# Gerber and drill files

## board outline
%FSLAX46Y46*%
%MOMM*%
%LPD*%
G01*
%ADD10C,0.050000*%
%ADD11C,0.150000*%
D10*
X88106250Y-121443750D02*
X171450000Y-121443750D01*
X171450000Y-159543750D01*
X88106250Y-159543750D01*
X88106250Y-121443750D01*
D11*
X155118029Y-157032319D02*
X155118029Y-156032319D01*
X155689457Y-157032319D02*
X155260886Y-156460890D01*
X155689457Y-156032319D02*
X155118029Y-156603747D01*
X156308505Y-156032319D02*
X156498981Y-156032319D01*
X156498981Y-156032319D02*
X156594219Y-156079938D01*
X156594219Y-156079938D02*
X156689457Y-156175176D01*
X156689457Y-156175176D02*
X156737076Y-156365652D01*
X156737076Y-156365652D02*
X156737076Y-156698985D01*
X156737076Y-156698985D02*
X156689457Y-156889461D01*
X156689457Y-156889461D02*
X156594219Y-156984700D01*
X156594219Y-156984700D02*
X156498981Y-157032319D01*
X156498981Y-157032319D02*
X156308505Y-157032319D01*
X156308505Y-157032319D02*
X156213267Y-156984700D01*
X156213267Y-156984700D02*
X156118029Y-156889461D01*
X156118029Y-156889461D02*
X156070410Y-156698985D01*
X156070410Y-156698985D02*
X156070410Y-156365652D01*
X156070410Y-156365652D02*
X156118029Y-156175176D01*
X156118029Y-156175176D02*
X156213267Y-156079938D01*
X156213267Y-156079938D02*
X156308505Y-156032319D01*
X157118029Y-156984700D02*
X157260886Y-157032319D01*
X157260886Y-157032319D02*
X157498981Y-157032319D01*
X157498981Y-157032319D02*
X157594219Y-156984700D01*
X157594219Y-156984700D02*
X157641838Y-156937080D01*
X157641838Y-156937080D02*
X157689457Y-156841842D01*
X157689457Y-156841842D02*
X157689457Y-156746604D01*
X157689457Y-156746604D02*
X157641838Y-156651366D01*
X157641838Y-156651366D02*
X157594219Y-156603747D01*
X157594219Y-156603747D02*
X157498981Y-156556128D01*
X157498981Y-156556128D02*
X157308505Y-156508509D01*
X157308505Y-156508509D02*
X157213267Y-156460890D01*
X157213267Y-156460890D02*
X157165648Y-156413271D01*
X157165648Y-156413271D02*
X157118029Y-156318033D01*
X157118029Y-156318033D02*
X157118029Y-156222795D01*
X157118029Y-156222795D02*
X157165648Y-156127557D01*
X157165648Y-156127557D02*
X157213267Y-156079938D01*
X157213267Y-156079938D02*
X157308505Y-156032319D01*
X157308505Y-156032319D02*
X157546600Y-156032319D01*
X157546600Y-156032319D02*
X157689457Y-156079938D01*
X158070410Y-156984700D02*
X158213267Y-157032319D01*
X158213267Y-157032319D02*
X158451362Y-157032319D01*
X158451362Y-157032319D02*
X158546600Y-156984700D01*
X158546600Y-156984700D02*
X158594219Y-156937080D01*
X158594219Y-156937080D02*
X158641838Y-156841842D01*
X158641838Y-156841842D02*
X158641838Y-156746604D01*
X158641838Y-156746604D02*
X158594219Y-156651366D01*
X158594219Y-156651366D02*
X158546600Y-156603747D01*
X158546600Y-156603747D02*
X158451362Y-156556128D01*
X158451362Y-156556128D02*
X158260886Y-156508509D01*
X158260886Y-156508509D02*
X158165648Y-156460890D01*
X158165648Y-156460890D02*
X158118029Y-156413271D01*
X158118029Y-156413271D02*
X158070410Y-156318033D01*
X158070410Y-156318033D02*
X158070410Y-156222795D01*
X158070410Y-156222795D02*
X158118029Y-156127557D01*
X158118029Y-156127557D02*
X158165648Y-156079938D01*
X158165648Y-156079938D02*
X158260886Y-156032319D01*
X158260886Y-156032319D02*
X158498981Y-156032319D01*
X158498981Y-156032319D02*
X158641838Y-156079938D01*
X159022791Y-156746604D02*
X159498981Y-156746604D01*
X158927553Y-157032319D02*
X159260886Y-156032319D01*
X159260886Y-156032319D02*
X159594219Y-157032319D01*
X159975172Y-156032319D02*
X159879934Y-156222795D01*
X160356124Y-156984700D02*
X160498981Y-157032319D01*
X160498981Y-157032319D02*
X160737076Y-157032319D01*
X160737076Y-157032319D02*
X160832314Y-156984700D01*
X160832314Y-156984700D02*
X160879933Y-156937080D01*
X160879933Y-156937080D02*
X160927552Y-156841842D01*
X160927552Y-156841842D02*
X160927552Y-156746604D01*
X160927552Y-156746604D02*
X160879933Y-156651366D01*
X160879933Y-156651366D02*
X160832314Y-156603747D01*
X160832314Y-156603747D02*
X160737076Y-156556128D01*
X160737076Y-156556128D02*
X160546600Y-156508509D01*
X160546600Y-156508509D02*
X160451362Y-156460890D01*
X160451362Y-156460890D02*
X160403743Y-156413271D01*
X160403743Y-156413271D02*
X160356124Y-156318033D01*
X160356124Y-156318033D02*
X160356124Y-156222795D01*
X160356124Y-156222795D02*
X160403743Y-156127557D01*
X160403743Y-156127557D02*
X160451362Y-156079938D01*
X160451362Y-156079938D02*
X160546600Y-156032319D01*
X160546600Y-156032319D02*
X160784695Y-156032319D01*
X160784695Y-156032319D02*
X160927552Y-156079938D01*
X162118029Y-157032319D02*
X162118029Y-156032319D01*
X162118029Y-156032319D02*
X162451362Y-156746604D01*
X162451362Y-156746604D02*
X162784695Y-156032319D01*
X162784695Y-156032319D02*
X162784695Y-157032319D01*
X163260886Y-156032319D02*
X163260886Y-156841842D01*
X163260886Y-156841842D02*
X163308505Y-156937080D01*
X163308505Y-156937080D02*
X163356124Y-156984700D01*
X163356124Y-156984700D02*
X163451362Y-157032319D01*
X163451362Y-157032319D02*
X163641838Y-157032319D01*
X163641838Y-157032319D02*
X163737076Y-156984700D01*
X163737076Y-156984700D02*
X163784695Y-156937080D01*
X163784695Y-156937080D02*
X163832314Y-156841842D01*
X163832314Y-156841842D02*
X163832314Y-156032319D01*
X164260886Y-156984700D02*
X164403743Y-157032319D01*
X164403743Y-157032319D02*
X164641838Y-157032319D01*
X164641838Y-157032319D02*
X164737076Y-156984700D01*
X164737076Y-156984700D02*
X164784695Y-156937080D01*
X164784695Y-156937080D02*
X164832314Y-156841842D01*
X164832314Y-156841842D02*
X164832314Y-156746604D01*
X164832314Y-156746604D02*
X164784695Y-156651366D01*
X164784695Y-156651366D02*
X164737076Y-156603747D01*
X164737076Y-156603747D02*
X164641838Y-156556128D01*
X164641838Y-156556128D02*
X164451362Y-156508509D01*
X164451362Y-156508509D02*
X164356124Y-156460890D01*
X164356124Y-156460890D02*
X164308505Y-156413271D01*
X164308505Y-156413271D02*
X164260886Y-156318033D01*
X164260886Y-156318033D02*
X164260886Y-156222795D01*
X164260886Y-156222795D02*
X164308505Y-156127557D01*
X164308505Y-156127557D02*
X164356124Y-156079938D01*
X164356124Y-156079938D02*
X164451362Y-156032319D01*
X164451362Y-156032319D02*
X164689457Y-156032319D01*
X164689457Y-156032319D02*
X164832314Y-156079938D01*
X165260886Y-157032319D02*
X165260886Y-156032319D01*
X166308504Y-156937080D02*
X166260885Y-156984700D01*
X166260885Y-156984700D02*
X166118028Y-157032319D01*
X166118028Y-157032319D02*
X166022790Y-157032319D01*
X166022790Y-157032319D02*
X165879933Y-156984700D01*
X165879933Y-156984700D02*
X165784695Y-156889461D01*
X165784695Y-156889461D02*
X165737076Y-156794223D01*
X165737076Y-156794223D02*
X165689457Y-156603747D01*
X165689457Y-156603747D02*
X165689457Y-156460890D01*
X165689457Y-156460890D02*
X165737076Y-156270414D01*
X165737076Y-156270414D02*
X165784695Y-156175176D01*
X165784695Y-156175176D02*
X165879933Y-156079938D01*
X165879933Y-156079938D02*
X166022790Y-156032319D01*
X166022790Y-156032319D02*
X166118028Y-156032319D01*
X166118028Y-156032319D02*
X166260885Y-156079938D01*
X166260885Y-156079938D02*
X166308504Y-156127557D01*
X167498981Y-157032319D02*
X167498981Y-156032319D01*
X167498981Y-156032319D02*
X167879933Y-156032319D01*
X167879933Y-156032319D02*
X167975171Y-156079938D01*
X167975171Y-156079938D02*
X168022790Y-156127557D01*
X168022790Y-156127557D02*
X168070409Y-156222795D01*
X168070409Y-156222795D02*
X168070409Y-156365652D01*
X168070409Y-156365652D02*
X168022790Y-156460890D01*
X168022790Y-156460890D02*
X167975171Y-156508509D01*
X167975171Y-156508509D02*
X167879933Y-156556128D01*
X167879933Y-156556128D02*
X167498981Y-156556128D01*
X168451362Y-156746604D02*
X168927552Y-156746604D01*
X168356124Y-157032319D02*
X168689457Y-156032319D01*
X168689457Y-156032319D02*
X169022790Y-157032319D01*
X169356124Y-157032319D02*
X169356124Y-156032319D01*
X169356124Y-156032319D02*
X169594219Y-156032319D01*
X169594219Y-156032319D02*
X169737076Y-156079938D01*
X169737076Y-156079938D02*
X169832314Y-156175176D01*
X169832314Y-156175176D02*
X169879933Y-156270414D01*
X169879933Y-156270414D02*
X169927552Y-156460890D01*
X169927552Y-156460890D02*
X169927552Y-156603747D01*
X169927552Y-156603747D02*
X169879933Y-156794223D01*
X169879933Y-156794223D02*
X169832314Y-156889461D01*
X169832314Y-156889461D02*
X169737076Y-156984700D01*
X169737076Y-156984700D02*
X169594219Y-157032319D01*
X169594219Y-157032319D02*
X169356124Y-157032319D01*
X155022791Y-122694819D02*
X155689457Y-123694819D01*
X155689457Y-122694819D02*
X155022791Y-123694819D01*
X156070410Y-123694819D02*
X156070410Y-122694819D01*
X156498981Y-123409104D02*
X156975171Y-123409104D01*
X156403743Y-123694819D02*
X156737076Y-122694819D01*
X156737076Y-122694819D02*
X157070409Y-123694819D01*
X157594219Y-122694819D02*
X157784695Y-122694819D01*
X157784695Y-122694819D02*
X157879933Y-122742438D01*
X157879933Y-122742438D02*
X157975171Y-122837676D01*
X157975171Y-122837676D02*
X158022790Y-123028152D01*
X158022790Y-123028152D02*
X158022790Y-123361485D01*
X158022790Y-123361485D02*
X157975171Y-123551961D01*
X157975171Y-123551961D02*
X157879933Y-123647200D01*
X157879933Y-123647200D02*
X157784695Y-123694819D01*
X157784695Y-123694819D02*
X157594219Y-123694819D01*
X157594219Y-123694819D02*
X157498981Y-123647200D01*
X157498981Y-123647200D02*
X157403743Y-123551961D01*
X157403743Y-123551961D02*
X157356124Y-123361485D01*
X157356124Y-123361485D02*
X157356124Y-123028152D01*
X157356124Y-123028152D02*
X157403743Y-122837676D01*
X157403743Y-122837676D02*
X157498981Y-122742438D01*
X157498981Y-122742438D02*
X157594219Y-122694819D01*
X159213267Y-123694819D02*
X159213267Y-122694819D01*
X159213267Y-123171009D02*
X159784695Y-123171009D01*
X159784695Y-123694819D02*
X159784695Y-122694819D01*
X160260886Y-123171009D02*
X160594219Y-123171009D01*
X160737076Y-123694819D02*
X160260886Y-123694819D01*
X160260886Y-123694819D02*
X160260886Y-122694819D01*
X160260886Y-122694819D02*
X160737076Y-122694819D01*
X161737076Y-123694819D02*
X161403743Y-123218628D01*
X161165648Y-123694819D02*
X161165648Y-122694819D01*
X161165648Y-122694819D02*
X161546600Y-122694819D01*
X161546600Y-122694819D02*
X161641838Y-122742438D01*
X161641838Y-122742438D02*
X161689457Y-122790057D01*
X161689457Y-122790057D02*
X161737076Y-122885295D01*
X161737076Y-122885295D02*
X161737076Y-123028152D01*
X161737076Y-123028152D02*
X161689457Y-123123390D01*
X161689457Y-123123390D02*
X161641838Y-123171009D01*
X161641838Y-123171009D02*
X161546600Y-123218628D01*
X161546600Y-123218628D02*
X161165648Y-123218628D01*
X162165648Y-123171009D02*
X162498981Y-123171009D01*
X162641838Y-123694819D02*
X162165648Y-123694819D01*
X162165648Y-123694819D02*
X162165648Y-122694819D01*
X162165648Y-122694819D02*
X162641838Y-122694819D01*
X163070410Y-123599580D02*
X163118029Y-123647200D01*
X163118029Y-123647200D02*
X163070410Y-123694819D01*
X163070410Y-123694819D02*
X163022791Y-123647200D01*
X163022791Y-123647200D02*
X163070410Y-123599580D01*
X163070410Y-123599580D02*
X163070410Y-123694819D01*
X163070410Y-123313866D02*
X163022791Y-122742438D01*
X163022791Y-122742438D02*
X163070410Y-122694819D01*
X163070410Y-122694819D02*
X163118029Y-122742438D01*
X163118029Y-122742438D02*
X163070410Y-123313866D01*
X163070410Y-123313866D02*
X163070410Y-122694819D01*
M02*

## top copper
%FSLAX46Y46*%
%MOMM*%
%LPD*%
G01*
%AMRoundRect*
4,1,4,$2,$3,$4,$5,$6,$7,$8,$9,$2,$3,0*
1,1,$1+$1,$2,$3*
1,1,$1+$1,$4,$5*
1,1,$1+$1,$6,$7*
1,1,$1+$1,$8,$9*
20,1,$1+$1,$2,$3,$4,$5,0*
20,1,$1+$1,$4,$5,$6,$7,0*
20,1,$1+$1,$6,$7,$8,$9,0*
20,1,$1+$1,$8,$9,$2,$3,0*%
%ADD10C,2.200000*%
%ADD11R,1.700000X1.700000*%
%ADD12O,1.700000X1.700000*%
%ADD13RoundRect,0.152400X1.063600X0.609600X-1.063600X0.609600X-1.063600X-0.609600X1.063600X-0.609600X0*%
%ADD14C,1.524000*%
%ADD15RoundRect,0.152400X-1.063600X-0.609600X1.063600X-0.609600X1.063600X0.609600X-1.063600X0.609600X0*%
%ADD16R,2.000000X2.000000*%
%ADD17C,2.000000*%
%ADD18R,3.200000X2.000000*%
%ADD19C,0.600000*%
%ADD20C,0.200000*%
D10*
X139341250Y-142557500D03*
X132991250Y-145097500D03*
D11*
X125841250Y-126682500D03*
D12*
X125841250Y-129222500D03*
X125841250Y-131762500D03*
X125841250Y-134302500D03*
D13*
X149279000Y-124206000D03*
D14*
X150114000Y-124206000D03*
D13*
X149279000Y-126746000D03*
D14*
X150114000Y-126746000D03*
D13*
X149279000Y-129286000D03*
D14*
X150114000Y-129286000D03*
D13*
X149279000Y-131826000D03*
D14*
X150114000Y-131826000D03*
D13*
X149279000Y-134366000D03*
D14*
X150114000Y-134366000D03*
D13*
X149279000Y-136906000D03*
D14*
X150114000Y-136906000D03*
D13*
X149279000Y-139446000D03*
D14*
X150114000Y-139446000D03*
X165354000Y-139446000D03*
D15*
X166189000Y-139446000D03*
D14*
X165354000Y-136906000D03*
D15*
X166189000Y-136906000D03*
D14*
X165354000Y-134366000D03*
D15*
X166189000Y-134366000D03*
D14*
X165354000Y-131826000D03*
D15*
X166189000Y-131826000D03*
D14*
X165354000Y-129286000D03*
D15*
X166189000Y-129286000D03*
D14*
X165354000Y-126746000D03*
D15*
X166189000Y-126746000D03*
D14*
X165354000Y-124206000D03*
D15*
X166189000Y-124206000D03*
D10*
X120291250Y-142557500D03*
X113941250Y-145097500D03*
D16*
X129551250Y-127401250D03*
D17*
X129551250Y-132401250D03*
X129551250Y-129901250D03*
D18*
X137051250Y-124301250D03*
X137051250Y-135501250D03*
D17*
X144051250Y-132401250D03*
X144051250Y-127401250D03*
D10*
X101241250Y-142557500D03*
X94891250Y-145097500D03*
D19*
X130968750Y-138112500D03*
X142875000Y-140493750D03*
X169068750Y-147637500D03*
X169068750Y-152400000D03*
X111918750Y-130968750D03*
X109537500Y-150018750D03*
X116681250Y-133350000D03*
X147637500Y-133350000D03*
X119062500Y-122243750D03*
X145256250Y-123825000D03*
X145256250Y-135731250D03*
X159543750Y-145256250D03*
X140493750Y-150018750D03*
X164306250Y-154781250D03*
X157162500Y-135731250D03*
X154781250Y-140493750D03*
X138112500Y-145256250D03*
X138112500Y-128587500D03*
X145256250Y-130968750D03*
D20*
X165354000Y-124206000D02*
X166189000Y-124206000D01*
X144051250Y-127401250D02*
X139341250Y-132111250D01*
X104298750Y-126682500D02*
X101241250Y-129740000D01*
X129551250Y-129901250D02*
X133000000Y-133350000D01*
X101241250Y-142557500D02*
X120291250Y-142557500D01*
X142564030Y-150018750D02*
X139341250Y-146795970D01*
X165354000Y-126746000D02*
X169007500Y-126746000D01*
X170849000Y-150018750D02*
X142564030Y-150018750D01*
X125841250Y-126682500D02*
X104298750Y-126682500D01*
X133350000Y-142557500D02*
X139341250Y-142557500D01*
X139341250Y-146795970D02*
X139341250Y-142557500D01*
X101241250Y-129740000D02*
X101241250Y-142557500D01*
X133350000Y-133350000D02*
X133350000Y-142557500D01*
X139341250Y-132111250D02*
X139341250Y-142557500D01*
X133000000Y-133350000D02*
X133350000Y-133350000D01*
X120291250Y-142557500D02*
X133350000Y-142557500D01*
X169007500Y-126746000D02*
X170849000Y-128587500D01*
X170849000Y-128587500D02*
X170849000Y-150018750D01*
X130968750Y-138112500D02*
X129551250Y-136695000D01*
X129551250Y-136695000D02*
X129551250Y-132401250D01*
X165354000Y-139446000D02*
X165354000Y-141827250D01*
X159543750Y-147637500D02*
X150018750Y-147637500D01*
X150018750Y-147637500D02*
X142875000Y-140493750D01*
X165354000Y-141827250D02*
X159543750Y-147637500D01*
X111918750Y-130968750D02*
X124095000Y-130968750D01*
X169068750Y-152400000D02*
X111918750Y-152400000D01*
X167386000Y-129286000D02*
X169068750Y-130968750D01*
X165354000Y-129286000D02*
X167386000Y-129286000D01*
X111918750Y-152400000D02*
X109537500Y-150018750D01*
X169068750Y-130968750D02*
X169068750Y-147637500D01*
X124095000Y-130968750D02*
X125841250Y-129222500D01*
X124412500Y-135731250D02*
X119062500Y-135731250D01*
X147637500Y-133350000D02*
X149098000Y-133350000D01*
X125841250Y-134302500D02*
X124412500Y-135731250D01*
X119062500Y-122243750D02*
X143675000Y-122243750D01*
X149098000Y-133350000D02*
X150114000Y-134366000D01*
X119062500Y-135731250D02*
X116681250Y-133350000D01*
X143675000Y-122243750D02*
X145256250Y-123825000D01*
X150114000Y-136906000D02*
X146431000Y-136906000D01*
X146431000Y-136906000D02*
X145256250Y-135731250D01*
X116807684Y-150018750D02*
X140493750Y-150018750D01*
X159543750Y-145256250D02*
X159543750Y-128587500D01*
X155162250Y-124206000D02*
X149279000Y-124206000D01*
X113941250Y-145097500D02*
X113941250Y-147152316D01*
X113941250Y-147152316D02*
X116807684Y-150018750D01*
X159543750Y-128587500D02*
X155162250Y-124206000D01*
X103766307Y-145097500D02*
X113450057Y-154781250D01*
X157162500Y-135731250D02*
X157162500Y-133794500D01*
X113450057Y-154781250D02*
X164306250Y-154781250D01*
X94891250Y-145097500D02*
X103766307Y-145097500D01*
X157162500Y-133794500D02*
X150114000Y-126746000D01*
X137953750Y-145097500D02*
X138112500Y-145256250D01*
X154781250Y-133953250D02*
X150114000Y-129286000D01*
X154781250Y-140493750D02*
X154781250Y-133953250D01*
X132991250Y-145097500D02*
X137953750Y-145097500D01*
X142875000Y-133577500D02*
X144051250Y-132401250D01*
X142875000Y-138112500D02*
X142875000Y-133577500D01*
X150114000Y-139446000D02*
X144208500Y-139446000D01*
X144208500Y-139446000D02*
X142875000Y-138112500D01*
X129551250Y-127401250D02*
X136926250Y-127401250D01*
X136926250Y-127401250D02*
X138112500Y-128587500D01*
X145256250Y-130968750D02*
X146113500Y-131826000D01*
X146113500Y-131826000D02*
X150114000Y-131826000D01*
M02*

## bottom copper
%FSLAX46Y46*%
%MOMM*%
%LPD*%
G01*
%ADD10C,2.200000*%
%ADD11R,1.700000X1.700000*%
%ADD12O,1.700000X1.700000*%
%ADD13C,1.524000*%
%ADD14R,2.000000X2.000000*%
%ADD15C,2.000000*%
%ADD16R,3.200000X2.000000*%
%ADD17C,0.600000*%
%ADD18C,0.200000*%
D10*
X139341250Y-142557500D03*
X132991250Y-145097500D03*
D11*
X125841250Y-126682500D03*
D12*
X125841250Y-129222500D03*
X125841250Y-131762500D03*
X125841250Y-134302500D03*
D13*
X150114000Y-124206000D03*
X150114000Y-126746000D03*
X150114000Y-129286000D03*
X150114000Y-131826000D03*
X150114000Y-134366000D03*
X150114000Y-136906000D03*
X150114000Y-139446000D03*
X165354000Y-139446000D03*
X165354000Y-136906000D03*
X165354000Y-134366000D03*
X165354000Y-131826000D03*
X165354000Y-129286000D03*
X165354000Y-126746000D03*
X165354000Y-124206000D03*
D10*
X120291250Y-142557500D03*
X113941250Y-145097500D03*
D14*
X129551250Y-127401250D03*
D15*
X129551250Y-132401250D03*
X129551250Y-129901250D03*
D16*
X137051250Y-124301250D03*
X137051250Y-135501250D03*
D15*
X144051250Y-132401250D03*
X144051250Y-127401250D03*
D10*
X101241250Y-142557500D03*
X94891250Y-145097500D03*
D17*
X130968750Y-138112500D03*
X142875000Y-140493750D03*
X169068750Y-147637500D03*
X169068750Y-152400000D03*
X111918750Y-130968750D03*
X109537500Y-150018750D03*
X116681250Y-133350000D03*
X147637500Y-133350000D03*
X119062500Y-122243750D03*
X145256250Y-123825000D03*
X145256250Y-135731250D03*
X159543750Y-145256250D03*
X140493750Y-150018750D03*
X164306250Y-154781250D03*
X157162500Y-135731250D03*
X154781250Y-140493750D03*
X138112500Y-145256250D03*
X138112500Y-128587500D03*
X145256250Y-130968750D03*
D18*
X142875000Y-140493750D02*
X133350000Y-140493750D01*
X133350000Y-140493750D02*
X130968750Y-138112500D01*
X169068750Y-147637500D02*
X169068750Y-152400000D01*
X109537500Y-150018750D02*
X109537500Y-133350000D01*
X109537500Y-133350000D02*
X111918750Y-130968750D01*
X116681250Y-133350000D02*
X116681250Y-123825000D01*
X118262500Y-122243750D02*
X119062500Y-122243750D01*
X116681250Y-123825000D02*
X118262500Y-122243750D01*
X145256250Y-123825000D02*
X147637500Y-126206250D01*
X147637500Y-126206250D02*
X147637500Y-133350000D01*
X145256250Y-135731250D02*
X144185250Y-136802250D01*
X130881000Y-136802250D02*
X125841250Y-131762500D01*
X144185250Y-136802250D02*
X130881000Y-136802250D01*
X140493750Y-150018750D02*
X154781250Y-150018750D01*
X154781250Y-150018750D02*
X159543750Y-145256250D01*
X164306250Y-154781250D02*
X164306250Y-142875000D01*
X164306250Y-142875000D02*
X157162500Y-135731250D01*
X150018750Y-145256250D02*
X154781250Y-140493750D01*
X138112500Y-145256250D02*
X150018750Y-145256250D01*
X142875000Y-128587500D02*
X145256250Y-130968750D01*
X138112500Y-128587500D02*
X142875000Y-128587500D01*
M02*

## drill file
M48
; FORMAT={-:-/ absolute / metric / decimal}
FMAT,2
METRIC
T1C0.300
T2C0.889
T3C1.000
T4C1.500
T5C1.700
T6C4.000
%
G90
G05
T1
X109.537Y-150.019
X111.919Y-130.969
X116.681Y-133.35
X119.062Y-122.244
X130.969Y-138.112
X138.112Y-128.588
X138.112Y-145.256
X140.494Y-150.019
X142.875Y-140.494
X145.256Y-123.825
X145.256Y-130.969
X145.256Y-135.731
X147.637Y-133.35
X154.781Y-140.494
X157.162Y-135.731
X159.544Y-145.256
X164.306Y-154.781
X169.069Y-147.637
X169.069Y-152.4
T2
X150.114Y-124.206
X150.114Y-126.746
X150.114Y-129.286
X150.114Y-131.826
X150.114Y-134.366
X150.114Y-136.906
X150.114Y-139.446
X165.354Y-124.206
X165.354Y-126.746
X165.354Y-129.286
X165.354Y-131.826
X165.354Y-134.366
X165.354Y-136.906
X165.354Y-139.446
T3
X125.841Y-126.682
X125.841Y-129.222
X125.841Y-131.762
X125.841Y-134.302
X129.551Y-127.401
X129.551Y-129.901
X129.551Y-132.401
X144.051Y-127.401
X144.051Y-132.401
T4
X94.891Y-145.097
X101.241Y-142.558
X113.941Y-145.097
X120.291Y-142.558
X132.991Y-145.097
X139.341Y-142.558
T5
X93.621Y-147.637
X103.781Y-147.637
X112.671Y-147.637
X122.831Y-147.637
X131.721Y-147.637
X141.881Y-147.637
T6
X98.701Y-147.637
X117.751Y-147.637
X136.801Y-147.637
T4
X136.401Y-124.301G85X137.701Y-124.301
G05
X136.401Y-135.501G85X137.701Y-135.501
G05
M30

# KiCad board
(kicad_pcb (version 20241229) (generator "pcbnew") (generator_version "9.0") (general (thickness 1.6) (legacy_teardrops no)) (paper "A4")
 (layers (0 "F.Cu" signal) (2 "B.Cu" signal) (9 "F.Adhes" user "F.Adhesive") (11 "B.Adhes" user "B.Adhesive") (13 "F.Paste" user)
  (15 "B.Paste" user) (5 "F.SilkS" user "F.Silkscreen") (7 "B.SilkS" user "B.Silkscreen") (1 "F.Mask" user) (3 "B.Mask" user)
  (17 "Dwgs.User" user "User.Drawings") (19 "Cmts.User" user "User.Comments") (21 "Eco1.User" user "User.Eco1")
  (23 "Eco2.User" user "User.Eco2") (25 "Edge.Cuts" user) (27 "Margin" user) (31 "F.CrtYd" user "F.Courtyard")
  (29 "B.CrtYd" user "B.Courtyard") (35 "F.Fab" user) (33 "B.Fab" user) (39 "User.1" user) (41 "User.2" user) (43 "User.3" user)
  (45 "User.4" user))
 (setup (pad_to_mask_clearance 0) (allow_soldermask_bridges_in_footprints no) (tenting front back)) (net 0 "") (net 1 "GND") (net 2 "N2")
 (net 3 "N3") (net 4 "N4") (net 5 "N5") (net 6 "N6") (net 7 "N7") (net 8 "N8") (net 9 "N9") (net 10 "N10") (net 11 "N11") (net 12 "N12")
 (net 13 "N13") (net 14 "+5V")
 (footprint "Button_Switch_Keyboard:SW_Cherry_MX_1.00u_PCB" (layer "F.Cu") (at 139.34125 142.5575)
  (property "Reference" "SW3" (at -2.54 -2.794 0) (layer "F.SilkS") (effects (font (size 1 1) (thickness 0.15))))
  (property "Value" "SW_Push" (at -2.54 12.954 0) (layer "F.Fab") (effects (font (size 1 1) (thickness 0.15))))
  (pad "" np_thru_hole circle (at -7.62 5.08) (size 1.7 1.7) (drill 1.7) (layers "*.Cu" "*.Mask"))
  (pad "" np_thru_hole circle (at -2.54 5.08) (size 4 4) (drill 4) (layers "*.Cu" "*.Mask"))
  (pad "" np_thru_hole circle (at 2.54 5.08) (size 1.7 1.7) (drill 1.7) (layers "*.Cu" "*.Mask"))
  (pad "1" thru_hole circle (at 0 0) (size 2.2 2.2) (drill 1.5) (layers "*.Cu" "*.Mask") (remove_unused_layers no) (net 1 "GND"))
  (pad "2" thru_hole circle (at -6.35 2.54) (size 2.2 2.2) (drill 1.5) (layers "*.Cu" "*.Mask") (remove_unused_layers no) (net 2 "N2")))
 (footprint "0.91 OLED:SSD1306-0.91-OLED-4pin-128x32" (layer "F.Cu") (at 89.34125 124.4925)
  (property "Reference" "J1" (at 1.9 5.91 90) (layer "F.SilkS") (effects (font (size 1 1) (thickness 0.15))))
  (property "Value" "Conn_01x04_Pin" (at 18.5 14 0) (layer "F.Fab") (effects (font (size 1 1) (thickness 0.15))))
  (pad "1" thru_hole rect (at 36.5 2.19) (size 1.7 1.7) (drill 1) (layers "*.Cu" "*.Mask") (remove_unused_layers no) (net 1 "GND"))
  (pad "2" thru_hole oval (at 36.5 4.73) (size 1.7 1.7) (drill 1) (layers "*.Cu" "*.Mask") (remove_unused_layers no) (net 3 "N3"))
  (pad "3" thru_hole oval (at 36.5 7.27) (size 1.7 1.7) (drill 1) (layers "*.Cu" "*.Mask") (remove_unused_layers no) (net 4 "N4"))
  (pad "4" thru_hole oval (at 36.5 9.81) (size 1.7 1.7) (drill 1) (layers "*.Cu" "*.Mask") (remove_unused_layers no) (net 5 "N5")))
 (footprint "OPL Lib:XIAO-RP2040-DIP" (layer "F.Cu") (at 157.734 131.826)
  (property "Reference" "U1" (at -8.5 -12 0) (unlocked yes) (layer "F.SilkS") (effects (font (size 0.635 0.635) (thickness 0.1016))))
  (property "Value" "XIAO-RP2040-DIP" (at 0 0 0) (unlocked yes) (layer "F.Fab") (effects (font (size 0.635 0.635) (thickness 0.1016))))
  (pad "1" smd roundrect (at -8.455 -7.62 180) (size 2.432 1.524) (layers "F.Cu" "F.Mask") (roundrect_rratio 0.1) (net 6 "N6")
   (thermal_bridge_angle 45))
  (pad "1" thru_hole circle (at -7.62 -7.62 180) (size 1.524 1.524) (drill 0.889) (layers "*.Cu" "*.Mask") (remove_unused_layers no)
   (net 6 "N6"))
  (pad "2" smd roundrect (at -8.455 -5.08 180) (size 2.432 1.524) (layers "F.Cu" "F.Mask") (roundrect_rratio 0.1) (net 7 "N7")
   (thermal_bridge_angle 45))
  (pad "2" thru_hole circle (at -7.62 -5.08 180) (size 1.524 1.524) (drill 0.889) (layers "*.Cu" "*.Mask") (remove_unused_layers no)
   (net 7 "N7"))
  (pad "3" smd roundrect (at -8.455 -2.54 180) (size 2.432 1.524) (layers "F.Cu" "F.Mask") (roundrect_rratio 0.1) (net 2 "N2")
   (thermal_bridge_angle 45))
  (pad "3" thru_hole circle (at -7.62 -2.54 180) (size 1.524 1.524) (drill 0.889) (layers "*.Cu" "*.Mask") (remove_unused_layers no)
   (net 2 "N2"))
  (pad "4" smd roundrect (at -8.455 0 180) (size 2.432 1.524) (layers "F.Cu" "F.Mask") (roundrect_rratio 0.1) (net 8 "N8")
   (thermal_bridge_angle 45))
  (pad "4" thru_hole circle (at -7.62 0 180) (size 1.524 1.524) (drill 0.889) (layers "*.Cu" "*.Mask") (remove_unused_layers no)
   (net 8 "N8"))
  (pad "5" smd roundrect (at -8.455 2.54 180) (size 2.432 1.524) (layers "F.Cu" "F.Mask") (roundrect_rratio 0.1) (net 5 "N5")
   (thermal_bridge_angle 45))
  (pad "5" thru_hole circle (at -7.62 2.54 180) (size 1.524 1.524) (drill 0.889) (layers "*.Cu" "*.Mask") (remove_unused_layers no)
   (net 5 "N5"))
  (pad "6" smd roundrect (at -8.455 5.08 180) (size 2.432 1.524) (layers "F.Cu" "F.Mask") (roundrect_rratio 0.1) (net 4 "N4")
   (thermal_bridge_angle 45))
  (pad "6" thru_hole circle (at -7.62 5.08 180) (size 1.524 1.524) (drill 0.889) (layers "*.Cu" "*.Mask") (remove_unused_layers no)
   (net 4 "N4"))
  (pad "7" smd roundrect (at -8.455 7.62 180) (size 2.432 1.524) (layers "F.Cu" "F.Mask") (roundrect_rratio 0.1) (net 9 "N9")
   (thermal_bridge_angle 45))
  (pad "7" thru_hole circle (at -7.62 7.62 180) (size 1.524 1.524) (drill 0.889) (layers "*.Cu" "*.Mask") (remove_unused_layers no)
   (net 9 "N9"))
  (pad "8" thru_hole circle (at 7.62 7.62) (size 1.524 1.524) (drill 0.889) (layers "*.Cu" "*.Mask") (remove_unused_layers no)
   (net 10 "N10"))
  (pad "8" smd roundrect (at 8.455 7.62) (size 2.432 1.524) (layers "F.Cu" "F.Mask") (roundrect_rratio 0.1) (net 10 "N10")
   (thermal_bridge_angle 45))
  (pad "9" thru_hole circle (at 7.62 5.08) (size 1.524 1.524) (drill 0.889) (layers "*.Cu" "*.Mask") (remove_unused_layers no)
   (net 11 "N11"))
  (pad "9" smd roundrect (at 8.455 5.08) (size 2.432 1.524) (layers "F.Cu" "F.Mask") (roundrect_rratio 0.1) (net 11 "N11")
   (thermal_bridge_angle 45))
  (pad "10" thru_hole circle (at 7.62 2.54) (size 1.524 1.524) (drill 0.889) (layers "*.Cu" "*.Mask") (remove_unused_layers no)
   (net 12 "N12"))
  (pad "10" smd roundrect (at 8.455 2.54) (size 2.432 1.524) (layers "F.Cu" "F.Mask") (roundrect_rratio 0.1) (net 12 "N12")
   (thermal_bridge_angle 45))
  (pad "11" thru_hole circle (at 7.62 0) (size 1.524 1.524) (drill 0.889) (layers "*.Cu" "*.Mask") (remove_unused_layers no) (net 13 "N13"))
  (pad "11" smd roundrect (at 8.455 0) (size 2.432 1.524) (layers "F.Cu" "F.Mask") (roundrect_rratio 0.1) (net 13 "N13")
   (thermal_bridge_angle 45))
  (pad "12" thru_hole circle (at 7.62 -2.54) (size 1.524 1.524) (drill 0.889) (layers "*.Cu" "*.Mask") (remove_unused_layers no)
   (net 3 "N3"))
  (pad "12" smd roundrect (at 8.455 -2.54) (size 2.432 1.524) (layers "F.Cu" "F.Mask") (roundrect_rratio 0.1) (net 3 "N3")
   (thermal_bridge_angle 45))
  (pad "13" thru_hole circle (at 7.62 -5.08) (size 1.524 1.524) (drill 0.889) (layers "*.Cu" "*.Mask") (remove_unused_layers no)
   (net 1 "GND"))
  (pad "13" smd roundrect (at 8.455 -5.08) (size 2.432 1.524) (layers "F.Cu" "F.Mask") (roundrect_rratio 0.1) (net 1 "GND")
   (thermal_bridge_angle 45))
  (pad "14" thru_hole circle (at 7.62 -7.62) (size 1.524 1.524) (drill 0.889) (layers "*.Cu" "*.Mask") (remove_unused_layers no)
   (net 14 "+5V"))
  (pad "14" smd roundrect (at 8.455 -7.62) (size 2.432 1.524) (layers "F.Cu" "F.Mask") (roundrect_rratio 0.1) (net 14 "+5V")
   (thermal_bridge_angle 45)))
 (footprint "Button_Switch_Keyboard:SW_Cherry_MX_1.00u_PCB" (layer "F.Cu") (at 120.29125 142.5575)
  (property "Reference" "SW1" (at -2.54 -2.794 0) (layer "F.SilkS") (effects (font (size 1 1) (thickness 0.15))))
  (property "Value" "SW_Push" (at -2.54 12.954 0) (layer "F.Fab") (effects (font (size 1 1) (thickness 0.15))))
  (pad "" np_thru_hole circle (at -7.62 5.08) (size 1.7 1.7) (drill 1.7) (layers "*.Cu" "*.Mask"))
  (pad "" np_thru_hole circle (at -2.54 5.08) (size 4 4) (drill 4) (layers "*.Cu" "*.Mask"))
  (pad "" np_thru_hole circle (at 2.54 5.08) (size 1.7 1.7) (drill 1.7) (layers "*.Cu" "*.Mask"))
  (pad "1" thru_hole circle (at 0 0) (size 2.2 2.2) (drill 1.5) (layers "*.Cu" "*.Mask") (remove_unused_layers no) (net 1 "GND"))
  (pad "2" thru_hole circle (at -6.35 2.54) (size 2.2 2.2) (drill 1.5) (layers "*.Cu" "*.Mask") (remove_unused_layers no) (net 6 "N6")))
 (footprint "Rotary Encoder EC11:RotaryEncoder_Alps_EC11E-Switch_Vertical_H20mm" (layer "F.Cu") (at 129.55125 127.40125)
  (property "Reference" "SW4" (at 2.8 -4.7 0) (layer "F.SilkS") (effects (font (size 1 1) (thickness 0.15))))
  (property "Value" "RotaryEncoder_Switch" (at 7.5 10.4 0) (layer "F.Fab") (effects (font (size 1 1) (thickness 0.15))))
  (pad "A" thru_hole rect (at 0 0) (size 2 2) (drill 1) (layers "*.Cu" "*.Mask") (remove_unused_layers no) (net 8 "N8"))
  (pad "B" thru_hole circle (at 0 5) (size 2 2) (drill 1) (layers "*.Cu" "*.Mask") (remove_unused_layers no) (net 10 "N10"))
  (pad "C" thru_hole circle (at 0 2.5) (size 2 2) (drill 1) (layers "*.Cu" "*.Mask") (remove_unused_layers no) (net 1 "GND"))
  (pad "MP" thru_hole rect (at 7.5 -3.1) (size 3.2 2) (drill oval 2.8 1.5) (layers "*.Cu" "*.Mask") (remove_unused_layers no))
  (pad "MP" thru_hole rect (at 7.5 8.1) (size 3.2 2) (drill oval 2.8 1.5) (layers "*.Cu" "*.Mask") (remove_unused_layers no))
  (pad "S1" thru_hole circle (at 14.5 5) (size 2 2) (drill 1) (layers "*.Cu" "*.Mask") (remove_unused_layers no) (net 9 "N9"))
  (pad "S2" thru_hole circle (at 14.5 0) (size 2 2) (drill 1) (layers "*.Cu" "*.Mask") (remove_unused_layers no) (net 1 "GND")))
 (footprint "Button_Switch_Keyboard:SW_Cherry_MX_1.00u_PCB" (layer "F.Cu") (at 101.24125 142.5575)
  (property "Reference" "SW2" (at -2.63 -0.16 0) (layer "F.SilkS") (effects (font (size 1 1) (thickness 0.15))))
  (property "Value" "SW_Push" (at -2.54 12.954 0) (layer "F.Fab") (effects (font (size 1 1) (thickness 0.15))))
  (pad "" np_thru_hole circle (at -7.62 5.08) (size 1.7 1.7) (drill 1.7) (layers "*.Cu" "*.Mask"))
  (pad "" np_thru_hole circle (at -2.54 5.08) (size 4 4) (drill 4) (layers "*.Cu" "*.Mask"))
  (pad "" np_thru_hole circle (at 2.54 5.08) (size 1.7 1.7) (drill 1.7) (layers "*.Cu" "*.Mask"))
  (pad "1" thru_hole circle (at 0 0) (size 2.2 2.2) (drill 1.5) (layers "*.Cu" "*.Mask") (remove_unused_layers no) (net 1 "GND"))
  (pad "2" thru_hole circle (at -6.35 2.54) (size 2.2 2.2) (drill 1.5) (layers "*.Cu" "*.Mask") (remove_unused_layers no) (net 7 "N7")))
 (gr_rect (start 88.10625 121.44375) (end 171.45 159.54375) (stroke (width 0.05) (type default)) (fill no) (layer "Edge.Cuts"))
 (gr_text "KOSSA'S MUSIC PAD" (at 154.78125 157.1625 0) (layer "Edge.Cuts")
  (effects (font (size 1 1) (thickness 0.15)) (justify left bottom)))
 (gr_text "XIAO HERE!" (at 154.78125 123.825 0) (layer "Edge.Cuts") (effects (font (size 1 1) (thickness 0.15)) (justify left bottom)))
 (segment (start 165.354 124.206) (end 166.189 124.206) (width 0.2) (layer "F.Cu") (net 14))
 (segment (start 144.05125 127.40125) (end 139.34125 132.11125) (width 0.2) (layer "F.Cu") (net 1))
 (segment (start 104.29875 126.6825) (end 101.24125 129.74) (width 0.2) (layer "F.Cu") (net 1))
 (segment (start 129.55125 129.90125) (end 133 133.35) (width 0.2) (layer "F.Cu") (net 1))
 (segment (start 101.24125 142.5575) (end 120.29125 142.5575) (width 0.2) (layer "F.Cu") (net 1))
 (segment (start 142.56403 150.01875) (end 139.34125 146.79597) (width 0.2) (layer "F.Cu") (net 1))
 (segment (start 165.354 126.746) (end 169.0075 126.746) (width 0.2) (layer "F.Cu") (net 1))
 (segment (start 170.849 150.01875) (end 142.56403 150.01875) (width 0.2) (layer "F.Cu") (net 1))
 (segment (start 125.84125 126.6825) (end 104.29875 126.6825) (width 0.2) (layer "F.Cu") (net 1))
 (segment (start 133.35 142.5575) (end 139.34125 142.5575) (width 0.2) (layer "F.Cu") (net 1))
 (segment (start 139.34125 146.79597) (end 139.34125 142.5575) (width 0.2) (layer "F.Cu") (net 1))
 (segment (start 101.24125 129.74) (end 101.24125 142.5575) (width 0.2) (layer "F.Cu") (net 1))
 (segment (start 133.35 133.35) (end 133.35 142.5575) (width 0.2) (layer "F.Cu") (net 1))
 (segment (start 139.34125 132.11125) (end 139.34125 142.5575) (width 0.2) (layer "F.Cu") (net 1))
 (segment (start 133 133.35) (end 133.35 133.35) (width 0.2) (layer "F.Cu") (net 1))
 (segment (start 120.29125 142.5575) (end 133.35 142.5575) (width 0.2) (layer "F.Cu") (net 1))
 (segment (start 169.0075 126.746) (end 170.849 128.5875) (width 0.2) (layer "F.Cu") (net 1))
 (segment (start 170.849 128.5875) (end 170.849 150.01875) (width 0.2) (layer "F.Cu") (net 1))
 (segment (start 130.96875 138.1125) (end 129.55125 136.695) (width 0.2) (layer "F.Cu") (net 10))
 (segment (start 129.55125 136.695) (end 129.55125 132.40125) (width 0.2) (layer "F.Cu") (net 10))
 (segment (start 165.354 139.446) (end 165.354 141.82725) (width 0.2) (layer "F.Cu") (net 10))
 (segment (start 159.54375 147.6375) (end 150.01875 147.6375) (width 0.2) (layer "F.Cu") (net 10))
 (segment (start 150.01875 147.6375) (end 142.875 140.49375) (width 0.2) (layer "F.Cu") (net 10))
 (segment (start 165.354 141.82725) (end 159.54375 147.6375) (width 0.2) (layer "F.Cu") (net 10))
 (via (at 130.96875 138.1125) (size 0.6) (drill 0.3) (layers "F.Cu" "B.Cu") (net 10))
 (via (at 142.875 140.49375) (size 0.6) (drill 0.3) (layers "F.Cu" "B.Cu") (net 10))
 (segment (start 142.875 140.49375) (end 133.35 140.49375) (width 0.2) (layer "B.Cu") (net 10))
 (segment (start 133.35 140.49375) (end 130.96875 138.1125) (width 0.2) (layer "B.Cu") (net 10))
 (segment (start 111.91875 130.96875) (end 124.095 130.96875) (width 0.2) (layer "F.Cu") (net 3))
 (segment (start 169.06875 152.4) (end 111.91875 152.4) (width 0.2) (layer "F.Cu") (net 3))
 (segment (start 167.386 129.286) (end 169.06875 130.96875) (width 0.2) (layer "F.Cu") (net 3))
 (segment (start 165.354 129.286) (end 167.386 129.286) (width 0.2) (layer "F.Cu") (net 3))
 (segment (start 111.91875 152.4) (end 109.5375 150.01875) (width 0.2) (layer "F.Cu") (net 3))
 (segment (start 169.06875 130.96875) (end 169.06875 147.6375) (width 0.2) (layer "F.Cu") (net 3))
 (segment (start 124.095 130.96875) (end 125.84125 129.2225) (width 0.2) (layer "F.Cu") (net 3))
 (via (at 169.06875 147.6375) (size 0.6) (drill 0.3) (layers "F.Cu" "B.Cu") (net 3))
 (via (at 169.06875 152.4) (size 0.6) (drill 0.3) (layers "F.Cu" "B.Cu") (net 3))
 (via (at 111.91875 130.96875) (size 0.6) (drill 0.3) (layers "F.Cu" "B.Cu") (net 3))
 (via (at 109.5375 150.01875) (size 0.6) (drill 0.3) (layers "F.Cu" "B.Cu") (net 3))
 (segment (start 169.06875 147.6375) (end 169.06875 152.4) (width 0.2) (layer "B.Cu") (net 3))
 (segment (start 109.5375 150.01875) (end 109.5375 133.35) (width 0.2) (layer "B.Cu") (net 3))
 (segment (start 109.5375 133.35) (end 111.91875 130.96875) (width 0.2) (layer "B.Cu") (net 3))
 (segment (start 124.4125 135.73125) (end 119.0625 135.73125) (width 0.2) (layer "F.Cu") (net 5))
 (segment (start 147.6375 133.35) (end 149.098 133.35) (width 0.2) (layer "F.Cu") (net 5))
 (segment (start 125.84125 134.3025) (end 124.4125 135.73125) (width 0.2) (layer "F.Cu") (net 5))
 (segment (start 119.0625 122.24375) (end 143.675 122.24375) (width 0.2) (layer "F.Cu") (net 5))
 (segment (start 149.098 133.35) (end 150.114 134.366) (width 0.2) (layer "F.Cu") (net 5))
 (segment (start 119.0625 135.73125) (end 116.68125 133.35) (width 0.2) (layer "F.Cu") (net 5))
 (segment (start 143.675 122.24375) (end 145.25625 123.825) (width 0.2) (layer "F.Cu") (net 5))
 (via (at 116.68125 133.35) (size 0.6) (drill 0.3) (layers "F.Cu" "B.Cu") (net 5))
 (via (at 147.6375 133.35) (size 0.6) (drill 0.3) (layers "F.Cu" "B.Cu") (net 5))
 (via (at 119.0625 122.24375) (size 0.6) (drill 0.3) (layers "F.Cu" "B.Cu") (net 5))
 (via (at 145.25625 123.825) (size 0.6) (drill 0.3) (layers "F.Cu" "B.Cu") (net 5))
 (segment (start 116.68125 133.35) (end 116.68125 123.825) (width 0.2) (layer "B.Cu") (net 5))
 (segment (start 118.2625 122.24375) (end 119.0625 122.24375) (width 0.2) (layer "B.Cu") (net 5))
 (segment (start 116.68125 123.825) (end 118.2625 122.24375) (width 0.2) (layer "B.Cu") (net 5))
 (segment (start 145.25625 123.825) (end 147.6375 126.20625) (width 0.2) (layer "B.Cu") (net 5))
 (segment (start 147.6375 126.20625) (end 147.6375 133.35) (width 0.2) (layer "B.Cu") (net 5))
 (segment (start 150.114 136.906) (end 146.431 136.906) (width 0.2) (layer "F.Cu") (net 4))
 (segment (start 146.431 136.906) (end 145.25625 135.73125) (width 0.2) (layer "F.Cu") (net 4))
 (via (at 145.25625 135.73125) (size 0.6) (drill 0.3) (layers "F.Cu" "B.Cu") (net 4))
 (segment (start 145.25625 135.73125) (end 144.18525 136.80225) (width 0.2) (layer "B.Cu") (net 4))
 (segment (start 130.881 136.80225) (end 125.84125 131.7625) (width 0.2) (layer "B.Cu") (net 4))
 (segment (start 144.18525 136.80225) (end 130.881 136.80225) (width 0.2) (layer "B.Cu") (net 4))
 (segment (start 116.807684 150.01875) (end 140.49375 150.01875) (width 0.2) (layer "F.Cu") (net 6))
 (segment (start 159.54375 145.25625) (end 159.54375 128.5875) (width 0.2) (layer "F.Cu") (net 6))
 (segment (start 155.16225 124.206) (end 149.279 124.206) (width 0.2) (layer "F.Cu") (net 6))
 (segment (start 113.94125 145.0975) (end 113.94125 147.152316) (width 0.2) (layer "F.Cu") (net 6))
 (segment (start 113.94125 147.152316) (end 116.807684 150.01875) (width 0.2) (layer "F.Cu") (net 6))
 (segment (start 159.54375 128.5875) (end 155.16225 124.206) (width 0.2) (layer "F.Cu") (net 6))
 (via (at 159.54375 145.25625) (size 0.6) (drill 0.3) (layers "F.Cu" "B.Cu") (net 6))
 (via (at 140.49375 150.01875) (size 0.6) (drill 0.3) (layers "F.Cu" "B.Cu") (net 6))
 (segment (start 140.49375 150.01875) (end 154.78125 150.01875) (width 0.2) (layer "B.Cu") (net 6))
 (segment (start 154.78125 150.01875) (end 159.54375 145.25625) (width 0.2) (layer "B.Cu") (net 6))
 (segment (start 103.766307 145.0975) (end 113.450057 154.78125) (width 0.2) (layer "F.Cu") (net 7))
 (segment (start 157.1625 135.73125) (end 157.1625 133.7945) (width 0.2) (layer "F.Cu") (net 7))
 (segment (start 113.450057 154.78125) (end 164.30625 154.78125) (width 0.2) (layer "F.Cu") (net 7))
 (segment (start 94.89125 145.0975) (end 103.766307 145.0975) (width 0.2) (layer "F.Cu") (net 7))
 (segment (start 157.1625 133.7945) (end 150.114 126.746) (width 0.2) (layer "F.Cu") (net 7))
 (via (at 164.30625 154.78125) (size 0.6) (drill 0.3) (layers "F.Cu" "B.Cu") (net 7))
 (via (at 157.1625 135.73125) (size 0.6) (drill 0.3) (layers "F.Cu" "B.Cu") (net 7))
 (segment (start 164.30625 154.78125) (end 164.30625 142.875) (width 0.2) (layer "B.Cu") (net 7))
 (segment (start 164.30625 142.875) (end 157.1625 135.73125) (width 0.2) (layer "B.Cu") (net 7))
 (segment (start 137.95375 145.0975) (end 138.1125 145.25625) (width 0.2) (layer "F.Cu") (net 2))
 (segment (start 154.78125 133.95325) (end 150.114 129.286) (width 0.2) (layer "F.Cu") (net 2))
 (segment (start 154.78125 140.49375) (end 154.78125 133.95325) (width 0.2) (layer "F.Cu") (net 2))
 (segment (start 132.99125 145.0975) (end 137.95375 145.0975) (width 0.2) (layer "F.Cu") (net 2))
 (via (at 154.78125 140.49375) (size 0.6) (drill 0.3) (layers "F.Cu" "B.Cu") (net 2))
 (via (at 138.1125 145.25625) (size 0.6) (drill 0.3) (layers "F.Cu" "B.Cu") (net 2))
 (segment (start 150.01875 145.25625) (end 154.78125 140.49375) (width 0.2) (layer "B.Cu") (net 2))
 (segment (start 138.1125 145.25625) (end 150.01875 145.25625) (width 0.2) (layer "B.Cu") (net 2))
 (segment (start 142.875 133.5775) (end 144.05125 132.40125) (width 0.2) (layer "F.Cu") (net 9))
 (segment (start 142.875 138.1125) (end 142.875 133.5775) (width 0.2) (layer "F.Cu") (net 9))
 (segment (start 150.114 139.446) (end 144.2085 139.446) (width 0.2) (layer "F.Cu") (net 9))
 (segment (start 144.2085 139.446) (end 142.875 138.1125) (width 0.2) (layer "F.Cu") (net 9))
 (segment (start 129.55125 127.40125) (end 136.92625 127.40125) (width 0.2) (layer "F.Cu") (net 8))
 (segment (start 136.92625 127.40125) (end 138.1125 128.5875) (width 0.2) (layer "F.Cu") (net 8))
 (segment (start 145.25625 130.96875) (end 146.1135 131.826) (width 0.2) (layer "F.Cu") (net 8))
 (segment (start 146.1135 131.826) (end 150.114 131.826) (width 0.2) (layer "F.Cu") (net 8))
 (via (at 138.1125 128.5875) (size 0.6) (drill 0.3) (layers "F.Cu" "B.Cu") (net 8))
 (via (at 145.25625 130.96875) (size 0.6) (drill 0.3) (layers "F.Cu" "B.Cu") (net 8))
 (segment (start 142.875 128.5875) (end 145.25625 130.96875) (width 0.2) (layer "B.Cu") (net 8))
 (segment (start 138.1125 128.5875) (end 142.875 128.5875) (width 0.2) (layer "B.Cu") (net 8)))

